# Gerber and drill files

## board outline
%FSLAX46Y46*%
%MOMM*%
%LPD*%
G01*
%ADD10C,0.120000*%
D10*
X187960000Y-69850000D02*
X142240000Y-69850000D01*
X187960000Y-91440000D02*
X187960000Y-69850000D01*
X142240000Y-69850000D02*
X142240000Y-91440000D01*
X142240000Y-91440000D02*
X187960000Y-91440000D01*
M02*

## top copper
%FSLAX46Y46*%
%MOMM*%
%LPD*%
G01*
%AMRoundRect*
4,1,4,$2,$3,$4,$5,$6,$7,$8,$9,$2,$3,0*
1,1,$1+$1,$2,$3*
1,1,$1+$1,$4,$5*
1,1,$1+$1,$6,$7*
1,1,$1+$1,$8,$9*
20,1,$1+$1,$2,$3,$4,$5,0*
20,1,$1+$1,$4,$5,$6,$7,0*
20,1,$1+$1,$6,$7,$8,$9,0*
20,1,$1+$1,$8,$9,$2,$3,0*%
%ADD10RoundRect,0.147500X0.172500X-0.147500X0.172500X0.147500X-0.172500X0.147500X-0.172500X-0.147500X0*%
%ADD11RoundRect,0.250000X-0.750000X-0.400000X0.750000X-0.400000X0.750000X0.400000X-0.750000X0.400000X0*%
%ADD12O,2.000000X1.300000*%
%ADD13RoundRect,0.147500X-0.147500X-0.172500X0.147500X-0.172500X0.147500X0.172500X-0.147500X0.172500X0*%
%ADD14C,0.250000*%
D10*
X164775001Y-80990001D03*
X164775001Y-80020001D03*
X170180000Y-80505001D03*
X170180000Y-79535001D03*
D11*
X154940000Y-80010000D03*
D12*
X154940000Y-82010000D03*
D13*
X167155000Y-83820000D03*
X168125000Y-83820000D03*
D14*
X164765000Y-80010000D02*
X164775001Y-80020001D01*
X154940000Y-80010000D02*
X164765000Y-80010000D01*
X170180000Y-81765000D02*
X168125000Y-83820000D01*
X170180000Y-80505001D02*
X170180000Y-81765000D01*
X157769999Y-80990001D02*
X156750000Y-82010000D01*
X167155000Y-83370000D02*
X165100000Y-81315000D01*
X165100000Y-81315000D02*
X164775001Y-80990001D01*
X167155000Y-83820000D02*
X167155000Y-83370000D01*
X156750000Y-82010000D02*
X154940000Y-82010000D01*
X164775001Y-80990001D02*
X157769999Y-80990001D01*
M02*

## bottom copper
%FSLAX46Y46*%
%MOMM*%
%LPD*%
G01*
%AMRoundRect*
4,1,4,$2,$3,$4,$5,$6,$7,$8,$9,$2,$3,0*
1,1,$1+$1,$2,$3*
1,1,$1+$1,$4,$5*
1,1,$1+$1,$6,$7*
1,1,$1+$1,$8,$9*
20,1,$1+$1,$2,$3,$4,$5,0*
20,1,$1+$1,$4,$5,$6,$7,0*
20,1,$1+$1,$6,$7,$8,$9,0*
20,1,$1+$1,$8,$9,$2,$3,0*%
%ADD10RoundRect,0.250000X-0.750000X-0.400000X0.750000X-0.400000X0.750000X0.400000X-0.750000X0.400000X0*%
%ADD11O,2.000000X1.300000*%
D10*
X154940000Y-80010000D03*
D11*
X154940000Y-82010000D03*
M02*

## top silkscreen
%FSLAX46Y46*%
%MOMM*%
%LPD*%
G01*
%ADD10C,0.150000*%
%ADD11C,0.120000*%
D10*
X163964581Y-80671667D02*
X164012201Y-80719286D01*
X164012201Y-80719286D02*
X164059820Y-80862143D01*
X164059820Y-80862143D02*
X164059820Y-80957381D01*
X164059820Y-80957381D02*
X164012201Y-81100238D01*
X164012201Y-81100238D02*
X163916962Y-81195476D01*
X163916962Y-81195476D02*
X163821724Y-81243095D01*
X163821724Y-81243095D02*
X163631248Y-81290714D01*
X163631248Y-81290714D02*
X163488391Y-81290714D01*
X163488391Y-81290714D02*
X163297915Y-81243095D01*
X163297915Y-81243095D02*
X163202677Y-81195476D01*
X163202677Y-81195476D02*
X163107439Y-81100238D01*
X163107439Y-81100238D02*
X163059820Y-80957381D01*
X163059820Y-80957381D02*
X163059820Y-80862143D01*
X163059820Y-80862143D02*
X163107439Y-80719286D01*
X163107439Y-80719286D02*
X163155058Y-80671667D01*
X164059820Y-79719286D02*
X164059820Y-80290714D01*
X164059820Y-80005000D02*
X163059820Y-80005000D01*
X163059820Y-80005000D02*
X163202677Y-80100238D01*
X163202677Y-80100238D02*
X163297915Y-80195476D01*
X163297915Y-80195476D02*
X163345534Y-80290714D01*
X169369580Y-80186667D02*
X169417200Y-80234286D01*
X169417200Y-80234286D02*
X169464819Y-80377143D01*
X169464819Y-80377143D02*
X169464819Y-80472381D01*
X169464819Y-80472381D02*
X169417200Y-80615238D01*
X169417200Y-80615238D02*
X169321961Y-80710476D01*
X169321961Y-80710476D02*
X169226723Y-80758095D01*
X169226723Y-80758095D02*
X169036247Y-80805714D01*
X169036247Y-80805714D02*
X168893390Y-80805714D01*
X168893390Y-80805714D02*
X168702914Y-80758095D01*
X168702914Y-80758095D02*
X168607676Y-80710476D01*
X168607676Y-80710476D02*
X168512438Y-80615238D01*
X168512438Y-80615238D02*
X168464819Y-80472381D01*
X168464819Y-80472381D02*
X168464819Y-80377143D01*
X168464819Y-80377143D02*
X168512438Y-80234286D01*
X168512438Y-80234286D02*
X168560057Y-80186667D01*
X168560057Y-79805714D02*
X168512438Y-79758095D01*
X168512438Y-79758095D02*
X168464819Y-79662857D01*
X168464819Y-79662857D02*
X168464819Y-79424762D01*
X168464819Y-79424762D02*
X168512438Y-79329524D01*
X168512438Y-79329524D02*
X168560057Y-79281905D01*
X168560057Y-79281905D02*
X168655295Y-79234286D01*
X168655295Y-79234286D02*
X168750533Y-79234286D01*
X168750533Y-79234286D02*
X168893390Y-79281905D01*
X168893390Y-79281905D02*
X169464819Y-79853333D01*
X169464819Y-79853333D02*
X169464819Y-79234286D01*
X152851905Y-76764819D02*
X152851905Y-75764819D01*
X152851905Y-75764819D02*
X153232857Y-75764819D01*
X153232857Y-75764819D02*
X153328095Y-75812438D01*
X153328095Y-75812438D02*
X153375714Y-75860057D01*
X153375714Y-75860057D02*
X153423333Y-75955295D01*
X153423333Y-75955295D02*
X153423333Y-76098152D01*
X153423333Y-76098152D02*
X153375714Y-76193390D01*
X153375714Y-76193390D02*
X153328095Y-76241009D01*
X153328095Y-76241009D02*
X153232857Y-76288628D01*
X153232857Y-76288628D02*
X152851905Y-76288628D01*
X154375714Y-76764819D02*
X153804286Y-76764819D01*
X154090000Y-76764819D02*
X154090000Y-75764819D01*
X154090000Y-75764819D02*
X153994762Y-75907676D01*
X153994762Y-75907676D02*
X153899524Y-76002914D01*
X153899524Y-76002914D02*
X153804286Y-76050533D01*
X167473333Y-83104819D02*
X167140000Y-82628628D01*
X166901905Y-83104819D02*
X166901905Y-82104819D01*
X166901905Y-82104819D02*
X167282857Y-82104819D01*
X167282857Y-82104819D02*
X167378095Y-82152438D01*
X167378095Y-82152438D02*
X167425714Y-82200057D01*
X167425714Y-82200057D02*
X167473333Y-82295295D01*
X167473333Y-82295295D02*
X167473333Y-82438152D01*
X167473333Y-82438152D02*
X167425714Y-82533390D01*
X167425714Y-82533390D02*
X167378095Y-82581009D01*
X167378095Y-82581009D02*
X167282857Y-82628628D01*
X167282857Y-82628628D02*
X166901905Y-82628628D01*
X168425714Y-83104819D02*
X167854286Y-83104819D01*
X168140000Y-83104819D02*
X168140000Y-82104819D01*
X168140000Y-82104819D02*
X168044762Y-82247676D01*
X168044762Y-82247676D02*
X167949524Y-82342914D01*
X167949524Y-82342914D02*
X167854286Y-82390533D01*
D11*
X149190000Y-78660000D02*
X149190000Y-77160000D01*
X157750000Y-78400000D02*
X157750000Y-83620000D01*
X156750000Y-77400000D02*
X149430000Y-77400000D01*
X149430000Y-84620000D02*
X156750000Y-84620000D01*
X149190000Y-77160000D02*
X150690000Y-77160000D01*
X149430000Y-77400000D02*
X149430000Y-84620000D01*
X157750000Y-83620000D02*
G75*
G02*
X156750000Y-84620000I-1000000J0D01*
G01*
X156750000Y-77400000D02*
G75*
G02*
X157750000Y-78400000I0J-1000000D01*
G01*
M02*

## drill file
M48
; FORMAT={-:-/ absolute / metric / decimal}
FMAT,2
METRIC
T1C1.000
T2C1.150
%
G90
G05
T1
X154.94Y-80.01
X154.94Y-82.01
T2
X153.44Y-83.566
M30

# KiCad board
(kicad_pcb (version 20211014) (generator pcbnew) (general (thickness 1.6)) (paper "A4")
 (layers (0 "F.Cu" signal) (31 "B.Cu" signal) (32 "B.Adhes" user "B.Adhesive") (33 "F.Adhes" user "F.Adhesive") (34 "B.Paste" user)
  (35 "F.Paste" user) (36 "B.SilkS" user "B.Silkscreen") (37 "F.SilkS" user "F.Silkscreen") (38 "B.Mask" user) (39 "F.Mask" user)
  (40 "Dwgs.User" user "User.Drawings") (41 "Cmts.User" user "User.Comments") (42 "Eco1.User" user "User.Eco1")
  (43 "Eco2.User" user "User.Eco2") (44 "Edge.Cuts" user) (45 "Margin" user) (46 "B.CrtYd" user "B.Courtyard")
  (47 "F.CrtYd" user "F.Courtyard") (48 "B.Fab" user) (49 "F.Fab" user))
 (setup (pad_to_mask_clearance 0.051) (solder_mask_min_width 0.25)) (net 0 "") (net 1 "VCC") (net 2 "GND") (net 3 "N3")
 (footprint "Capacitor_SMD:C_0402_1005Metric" (layer "F.Cu") (at 164.775001 80.505001 90)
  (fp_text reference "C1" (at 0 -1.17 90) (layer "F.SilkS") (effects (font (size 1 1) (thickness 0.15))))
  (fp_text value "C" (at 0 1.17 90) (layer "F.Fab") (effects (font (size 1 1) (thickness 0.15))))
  (pad "1" smd roundrect locked (at -0.485 0 90) (size 0.59 0.64) (layers "F.Cu" "F.Paste" "F.Mask") (roundrect_rratio 0.25) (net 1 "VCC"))
  (pad "2" smd roundrect locked (at 0.485 0 90) (size 0.59 0.64) (layers "F.Cu" "F.Paste" "F.Mask") (roundrect_rratio 0.25) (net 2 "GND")))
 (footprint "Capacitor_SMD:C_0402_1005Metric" (layer "F.Cu") (at 170.18 80.020001 90)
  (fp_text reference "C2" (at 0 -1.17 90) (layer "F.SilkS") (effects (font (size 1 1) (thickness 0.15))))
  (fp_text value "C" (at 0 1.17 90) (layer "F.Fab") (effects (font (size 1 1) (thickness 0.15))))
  (pad "1" smd roundrect locked (at -0.485 0 90) (size 0.59 0.64) (layers "F.Cu" "F.Paste" "F.Mask") (roundrect_rratio 0.25) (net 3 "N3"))
  (pad "2" smd roundrect locked (at 0.485 0 90) (size 0.59 0.64) (layers "F.Cu" "F.Paste" "F.Mask") (roundrect_rratio 0.25) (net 2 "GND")))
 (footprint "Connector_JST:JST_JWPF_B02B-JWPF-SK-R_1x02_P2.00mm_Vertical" (layer "F.Cu") (at 154.94 80.01)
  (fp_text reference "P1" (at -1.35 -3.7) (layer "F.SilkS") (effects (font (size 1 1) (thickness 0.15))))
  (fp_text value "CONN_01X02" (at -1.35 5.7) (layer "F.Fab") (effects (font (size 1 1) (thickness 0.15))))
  (fp_line (start -5.75 -1.35) (end -5.75 -2.85) (layer "F.SilkS") (width 0.12))
  (fp_line (start 2.81 -1.61) (end 2.81 3.61) (layer "F.SilkS") (width 0.12))
  (fp_line (start 1.81 -2.61) (end -5.51 -2.61) (layer "F.SilkS") (width 0.12))
  (fp_line (start -5.51 4.61) (end 1.81 4.61) (layer "F.SilkS") (width 0.12))
  (fp_line (start -5.75 -2.85) (end -4.25 -2.85) (layer "F.SilkS") (width 0.12))
  (fp_line (start -5.51 -2.61) (end -5.51 4.61) (layer "F.SilkS") (width 0.12))
  (fp_arc (start 2.81 3.61) (mid 2.517107 4.317107) (end 1.81 4.61) (layer "F.SilkS") (width 0.12))
  (fp_arc (start 1.81 -2.61) (mid 2.517107 -2.317107) (end 2.81 -1.61) (layer "F.SilkS") (width 0.12))
  (pad "" np_thru_hole circle (at -1.5 3.556) (size 1.15 1.15) (drill 1.15) (layers *.Cu *.Mask))
  (pad "1" thru_hole roundrect (at 0 0) (size 2 1.3) (drill 1) (layers *.Cu *.Mask) (roundrect_rratio 0.192308) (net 2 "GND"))
  (pad "2" thru_hole oval (at 0 2) (size 2 1.3) (drill 1) (layers *.Cu *.Mask) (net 1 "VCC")))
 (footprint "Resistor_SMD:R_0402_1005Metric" (layer "F.Cu") (at 167.64 83.82)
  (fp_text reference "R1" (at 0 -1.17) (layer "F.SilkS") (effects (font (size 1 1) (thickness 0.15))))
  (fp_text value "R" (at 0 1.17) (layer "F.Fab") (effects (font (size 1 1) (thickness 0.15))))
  (pad "1" smd roundrect locked (at -0.485 0) (size 0.59 0.64) (layers "F.Cu" "F.Paste" "F.Mask") (roundrect_rratio 0.25) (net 1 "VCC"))
  (pad "2" smd roundrect locked (at 0.485 0) (size 0.59 0.64) (layers "F.Cu" "F.Paste" "F.Mask") (roundrect_rratio 0.25) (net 3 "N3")))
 (gr_line (start 187.96 69.85) (end 142.24 69.85) (layer "Edge.Cuts") (width 0.12))
 (gr_line (start 187.96 91.44) (end 187.96 69.85) (layer "Edge.Cuts") (width 0.12))
 (gr_line (start 142.24 69.85) (end 142.24 91.44) (layer "Edge.Cuts") (width 0.12))
 (gr_line (start 142.24 91.44) (end 187.96 91.44) (layer "Edge.Cuts") (width 0.12))
 (segment (start 164.765 80.01) (end 164.775001 80.020001) (width 0.25) (layer "F.Cu") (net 2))
 (segment (start 154.94 80.01) (end 164.765 80.01) (width 0.25) (layer "F.Cu") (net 2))
 (segment (start 170.18 81.765) (end 168.125 83.82) (width 0.25) (layer "F.Cu") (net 3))
 (segment (start 170.18 80.505001) (end 170.18 81.765) (width 0.25) (layer "F.Cu") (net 3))
 (segment (start 157.769999 80.990001) (end 156.75 82.01) (width 0.25) (layer "F.Cu") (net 1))
 (segment (start 167.155 83.37) (end 165.1 81.315) (width 0.25) (layer "F.Cu") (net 1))
 (segment (start 165.1 81.315) (end 164.775001 80.990001) (width 0.25) (layer "F.Cu") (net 1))
 (segment (start 167.155 83.82) (end 167.155 83.37) (width 0.25) (layer "F.Cu") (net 1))
 (segment (start 156.75 82.01) (end 154.94 82.01) (width 0.25) (layer "F.Cu") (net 1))
 (segment (start 164.775001 80.990001) (end 157.769999 80.990001) (width 0.25) (layer "F.Cu") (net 1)))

